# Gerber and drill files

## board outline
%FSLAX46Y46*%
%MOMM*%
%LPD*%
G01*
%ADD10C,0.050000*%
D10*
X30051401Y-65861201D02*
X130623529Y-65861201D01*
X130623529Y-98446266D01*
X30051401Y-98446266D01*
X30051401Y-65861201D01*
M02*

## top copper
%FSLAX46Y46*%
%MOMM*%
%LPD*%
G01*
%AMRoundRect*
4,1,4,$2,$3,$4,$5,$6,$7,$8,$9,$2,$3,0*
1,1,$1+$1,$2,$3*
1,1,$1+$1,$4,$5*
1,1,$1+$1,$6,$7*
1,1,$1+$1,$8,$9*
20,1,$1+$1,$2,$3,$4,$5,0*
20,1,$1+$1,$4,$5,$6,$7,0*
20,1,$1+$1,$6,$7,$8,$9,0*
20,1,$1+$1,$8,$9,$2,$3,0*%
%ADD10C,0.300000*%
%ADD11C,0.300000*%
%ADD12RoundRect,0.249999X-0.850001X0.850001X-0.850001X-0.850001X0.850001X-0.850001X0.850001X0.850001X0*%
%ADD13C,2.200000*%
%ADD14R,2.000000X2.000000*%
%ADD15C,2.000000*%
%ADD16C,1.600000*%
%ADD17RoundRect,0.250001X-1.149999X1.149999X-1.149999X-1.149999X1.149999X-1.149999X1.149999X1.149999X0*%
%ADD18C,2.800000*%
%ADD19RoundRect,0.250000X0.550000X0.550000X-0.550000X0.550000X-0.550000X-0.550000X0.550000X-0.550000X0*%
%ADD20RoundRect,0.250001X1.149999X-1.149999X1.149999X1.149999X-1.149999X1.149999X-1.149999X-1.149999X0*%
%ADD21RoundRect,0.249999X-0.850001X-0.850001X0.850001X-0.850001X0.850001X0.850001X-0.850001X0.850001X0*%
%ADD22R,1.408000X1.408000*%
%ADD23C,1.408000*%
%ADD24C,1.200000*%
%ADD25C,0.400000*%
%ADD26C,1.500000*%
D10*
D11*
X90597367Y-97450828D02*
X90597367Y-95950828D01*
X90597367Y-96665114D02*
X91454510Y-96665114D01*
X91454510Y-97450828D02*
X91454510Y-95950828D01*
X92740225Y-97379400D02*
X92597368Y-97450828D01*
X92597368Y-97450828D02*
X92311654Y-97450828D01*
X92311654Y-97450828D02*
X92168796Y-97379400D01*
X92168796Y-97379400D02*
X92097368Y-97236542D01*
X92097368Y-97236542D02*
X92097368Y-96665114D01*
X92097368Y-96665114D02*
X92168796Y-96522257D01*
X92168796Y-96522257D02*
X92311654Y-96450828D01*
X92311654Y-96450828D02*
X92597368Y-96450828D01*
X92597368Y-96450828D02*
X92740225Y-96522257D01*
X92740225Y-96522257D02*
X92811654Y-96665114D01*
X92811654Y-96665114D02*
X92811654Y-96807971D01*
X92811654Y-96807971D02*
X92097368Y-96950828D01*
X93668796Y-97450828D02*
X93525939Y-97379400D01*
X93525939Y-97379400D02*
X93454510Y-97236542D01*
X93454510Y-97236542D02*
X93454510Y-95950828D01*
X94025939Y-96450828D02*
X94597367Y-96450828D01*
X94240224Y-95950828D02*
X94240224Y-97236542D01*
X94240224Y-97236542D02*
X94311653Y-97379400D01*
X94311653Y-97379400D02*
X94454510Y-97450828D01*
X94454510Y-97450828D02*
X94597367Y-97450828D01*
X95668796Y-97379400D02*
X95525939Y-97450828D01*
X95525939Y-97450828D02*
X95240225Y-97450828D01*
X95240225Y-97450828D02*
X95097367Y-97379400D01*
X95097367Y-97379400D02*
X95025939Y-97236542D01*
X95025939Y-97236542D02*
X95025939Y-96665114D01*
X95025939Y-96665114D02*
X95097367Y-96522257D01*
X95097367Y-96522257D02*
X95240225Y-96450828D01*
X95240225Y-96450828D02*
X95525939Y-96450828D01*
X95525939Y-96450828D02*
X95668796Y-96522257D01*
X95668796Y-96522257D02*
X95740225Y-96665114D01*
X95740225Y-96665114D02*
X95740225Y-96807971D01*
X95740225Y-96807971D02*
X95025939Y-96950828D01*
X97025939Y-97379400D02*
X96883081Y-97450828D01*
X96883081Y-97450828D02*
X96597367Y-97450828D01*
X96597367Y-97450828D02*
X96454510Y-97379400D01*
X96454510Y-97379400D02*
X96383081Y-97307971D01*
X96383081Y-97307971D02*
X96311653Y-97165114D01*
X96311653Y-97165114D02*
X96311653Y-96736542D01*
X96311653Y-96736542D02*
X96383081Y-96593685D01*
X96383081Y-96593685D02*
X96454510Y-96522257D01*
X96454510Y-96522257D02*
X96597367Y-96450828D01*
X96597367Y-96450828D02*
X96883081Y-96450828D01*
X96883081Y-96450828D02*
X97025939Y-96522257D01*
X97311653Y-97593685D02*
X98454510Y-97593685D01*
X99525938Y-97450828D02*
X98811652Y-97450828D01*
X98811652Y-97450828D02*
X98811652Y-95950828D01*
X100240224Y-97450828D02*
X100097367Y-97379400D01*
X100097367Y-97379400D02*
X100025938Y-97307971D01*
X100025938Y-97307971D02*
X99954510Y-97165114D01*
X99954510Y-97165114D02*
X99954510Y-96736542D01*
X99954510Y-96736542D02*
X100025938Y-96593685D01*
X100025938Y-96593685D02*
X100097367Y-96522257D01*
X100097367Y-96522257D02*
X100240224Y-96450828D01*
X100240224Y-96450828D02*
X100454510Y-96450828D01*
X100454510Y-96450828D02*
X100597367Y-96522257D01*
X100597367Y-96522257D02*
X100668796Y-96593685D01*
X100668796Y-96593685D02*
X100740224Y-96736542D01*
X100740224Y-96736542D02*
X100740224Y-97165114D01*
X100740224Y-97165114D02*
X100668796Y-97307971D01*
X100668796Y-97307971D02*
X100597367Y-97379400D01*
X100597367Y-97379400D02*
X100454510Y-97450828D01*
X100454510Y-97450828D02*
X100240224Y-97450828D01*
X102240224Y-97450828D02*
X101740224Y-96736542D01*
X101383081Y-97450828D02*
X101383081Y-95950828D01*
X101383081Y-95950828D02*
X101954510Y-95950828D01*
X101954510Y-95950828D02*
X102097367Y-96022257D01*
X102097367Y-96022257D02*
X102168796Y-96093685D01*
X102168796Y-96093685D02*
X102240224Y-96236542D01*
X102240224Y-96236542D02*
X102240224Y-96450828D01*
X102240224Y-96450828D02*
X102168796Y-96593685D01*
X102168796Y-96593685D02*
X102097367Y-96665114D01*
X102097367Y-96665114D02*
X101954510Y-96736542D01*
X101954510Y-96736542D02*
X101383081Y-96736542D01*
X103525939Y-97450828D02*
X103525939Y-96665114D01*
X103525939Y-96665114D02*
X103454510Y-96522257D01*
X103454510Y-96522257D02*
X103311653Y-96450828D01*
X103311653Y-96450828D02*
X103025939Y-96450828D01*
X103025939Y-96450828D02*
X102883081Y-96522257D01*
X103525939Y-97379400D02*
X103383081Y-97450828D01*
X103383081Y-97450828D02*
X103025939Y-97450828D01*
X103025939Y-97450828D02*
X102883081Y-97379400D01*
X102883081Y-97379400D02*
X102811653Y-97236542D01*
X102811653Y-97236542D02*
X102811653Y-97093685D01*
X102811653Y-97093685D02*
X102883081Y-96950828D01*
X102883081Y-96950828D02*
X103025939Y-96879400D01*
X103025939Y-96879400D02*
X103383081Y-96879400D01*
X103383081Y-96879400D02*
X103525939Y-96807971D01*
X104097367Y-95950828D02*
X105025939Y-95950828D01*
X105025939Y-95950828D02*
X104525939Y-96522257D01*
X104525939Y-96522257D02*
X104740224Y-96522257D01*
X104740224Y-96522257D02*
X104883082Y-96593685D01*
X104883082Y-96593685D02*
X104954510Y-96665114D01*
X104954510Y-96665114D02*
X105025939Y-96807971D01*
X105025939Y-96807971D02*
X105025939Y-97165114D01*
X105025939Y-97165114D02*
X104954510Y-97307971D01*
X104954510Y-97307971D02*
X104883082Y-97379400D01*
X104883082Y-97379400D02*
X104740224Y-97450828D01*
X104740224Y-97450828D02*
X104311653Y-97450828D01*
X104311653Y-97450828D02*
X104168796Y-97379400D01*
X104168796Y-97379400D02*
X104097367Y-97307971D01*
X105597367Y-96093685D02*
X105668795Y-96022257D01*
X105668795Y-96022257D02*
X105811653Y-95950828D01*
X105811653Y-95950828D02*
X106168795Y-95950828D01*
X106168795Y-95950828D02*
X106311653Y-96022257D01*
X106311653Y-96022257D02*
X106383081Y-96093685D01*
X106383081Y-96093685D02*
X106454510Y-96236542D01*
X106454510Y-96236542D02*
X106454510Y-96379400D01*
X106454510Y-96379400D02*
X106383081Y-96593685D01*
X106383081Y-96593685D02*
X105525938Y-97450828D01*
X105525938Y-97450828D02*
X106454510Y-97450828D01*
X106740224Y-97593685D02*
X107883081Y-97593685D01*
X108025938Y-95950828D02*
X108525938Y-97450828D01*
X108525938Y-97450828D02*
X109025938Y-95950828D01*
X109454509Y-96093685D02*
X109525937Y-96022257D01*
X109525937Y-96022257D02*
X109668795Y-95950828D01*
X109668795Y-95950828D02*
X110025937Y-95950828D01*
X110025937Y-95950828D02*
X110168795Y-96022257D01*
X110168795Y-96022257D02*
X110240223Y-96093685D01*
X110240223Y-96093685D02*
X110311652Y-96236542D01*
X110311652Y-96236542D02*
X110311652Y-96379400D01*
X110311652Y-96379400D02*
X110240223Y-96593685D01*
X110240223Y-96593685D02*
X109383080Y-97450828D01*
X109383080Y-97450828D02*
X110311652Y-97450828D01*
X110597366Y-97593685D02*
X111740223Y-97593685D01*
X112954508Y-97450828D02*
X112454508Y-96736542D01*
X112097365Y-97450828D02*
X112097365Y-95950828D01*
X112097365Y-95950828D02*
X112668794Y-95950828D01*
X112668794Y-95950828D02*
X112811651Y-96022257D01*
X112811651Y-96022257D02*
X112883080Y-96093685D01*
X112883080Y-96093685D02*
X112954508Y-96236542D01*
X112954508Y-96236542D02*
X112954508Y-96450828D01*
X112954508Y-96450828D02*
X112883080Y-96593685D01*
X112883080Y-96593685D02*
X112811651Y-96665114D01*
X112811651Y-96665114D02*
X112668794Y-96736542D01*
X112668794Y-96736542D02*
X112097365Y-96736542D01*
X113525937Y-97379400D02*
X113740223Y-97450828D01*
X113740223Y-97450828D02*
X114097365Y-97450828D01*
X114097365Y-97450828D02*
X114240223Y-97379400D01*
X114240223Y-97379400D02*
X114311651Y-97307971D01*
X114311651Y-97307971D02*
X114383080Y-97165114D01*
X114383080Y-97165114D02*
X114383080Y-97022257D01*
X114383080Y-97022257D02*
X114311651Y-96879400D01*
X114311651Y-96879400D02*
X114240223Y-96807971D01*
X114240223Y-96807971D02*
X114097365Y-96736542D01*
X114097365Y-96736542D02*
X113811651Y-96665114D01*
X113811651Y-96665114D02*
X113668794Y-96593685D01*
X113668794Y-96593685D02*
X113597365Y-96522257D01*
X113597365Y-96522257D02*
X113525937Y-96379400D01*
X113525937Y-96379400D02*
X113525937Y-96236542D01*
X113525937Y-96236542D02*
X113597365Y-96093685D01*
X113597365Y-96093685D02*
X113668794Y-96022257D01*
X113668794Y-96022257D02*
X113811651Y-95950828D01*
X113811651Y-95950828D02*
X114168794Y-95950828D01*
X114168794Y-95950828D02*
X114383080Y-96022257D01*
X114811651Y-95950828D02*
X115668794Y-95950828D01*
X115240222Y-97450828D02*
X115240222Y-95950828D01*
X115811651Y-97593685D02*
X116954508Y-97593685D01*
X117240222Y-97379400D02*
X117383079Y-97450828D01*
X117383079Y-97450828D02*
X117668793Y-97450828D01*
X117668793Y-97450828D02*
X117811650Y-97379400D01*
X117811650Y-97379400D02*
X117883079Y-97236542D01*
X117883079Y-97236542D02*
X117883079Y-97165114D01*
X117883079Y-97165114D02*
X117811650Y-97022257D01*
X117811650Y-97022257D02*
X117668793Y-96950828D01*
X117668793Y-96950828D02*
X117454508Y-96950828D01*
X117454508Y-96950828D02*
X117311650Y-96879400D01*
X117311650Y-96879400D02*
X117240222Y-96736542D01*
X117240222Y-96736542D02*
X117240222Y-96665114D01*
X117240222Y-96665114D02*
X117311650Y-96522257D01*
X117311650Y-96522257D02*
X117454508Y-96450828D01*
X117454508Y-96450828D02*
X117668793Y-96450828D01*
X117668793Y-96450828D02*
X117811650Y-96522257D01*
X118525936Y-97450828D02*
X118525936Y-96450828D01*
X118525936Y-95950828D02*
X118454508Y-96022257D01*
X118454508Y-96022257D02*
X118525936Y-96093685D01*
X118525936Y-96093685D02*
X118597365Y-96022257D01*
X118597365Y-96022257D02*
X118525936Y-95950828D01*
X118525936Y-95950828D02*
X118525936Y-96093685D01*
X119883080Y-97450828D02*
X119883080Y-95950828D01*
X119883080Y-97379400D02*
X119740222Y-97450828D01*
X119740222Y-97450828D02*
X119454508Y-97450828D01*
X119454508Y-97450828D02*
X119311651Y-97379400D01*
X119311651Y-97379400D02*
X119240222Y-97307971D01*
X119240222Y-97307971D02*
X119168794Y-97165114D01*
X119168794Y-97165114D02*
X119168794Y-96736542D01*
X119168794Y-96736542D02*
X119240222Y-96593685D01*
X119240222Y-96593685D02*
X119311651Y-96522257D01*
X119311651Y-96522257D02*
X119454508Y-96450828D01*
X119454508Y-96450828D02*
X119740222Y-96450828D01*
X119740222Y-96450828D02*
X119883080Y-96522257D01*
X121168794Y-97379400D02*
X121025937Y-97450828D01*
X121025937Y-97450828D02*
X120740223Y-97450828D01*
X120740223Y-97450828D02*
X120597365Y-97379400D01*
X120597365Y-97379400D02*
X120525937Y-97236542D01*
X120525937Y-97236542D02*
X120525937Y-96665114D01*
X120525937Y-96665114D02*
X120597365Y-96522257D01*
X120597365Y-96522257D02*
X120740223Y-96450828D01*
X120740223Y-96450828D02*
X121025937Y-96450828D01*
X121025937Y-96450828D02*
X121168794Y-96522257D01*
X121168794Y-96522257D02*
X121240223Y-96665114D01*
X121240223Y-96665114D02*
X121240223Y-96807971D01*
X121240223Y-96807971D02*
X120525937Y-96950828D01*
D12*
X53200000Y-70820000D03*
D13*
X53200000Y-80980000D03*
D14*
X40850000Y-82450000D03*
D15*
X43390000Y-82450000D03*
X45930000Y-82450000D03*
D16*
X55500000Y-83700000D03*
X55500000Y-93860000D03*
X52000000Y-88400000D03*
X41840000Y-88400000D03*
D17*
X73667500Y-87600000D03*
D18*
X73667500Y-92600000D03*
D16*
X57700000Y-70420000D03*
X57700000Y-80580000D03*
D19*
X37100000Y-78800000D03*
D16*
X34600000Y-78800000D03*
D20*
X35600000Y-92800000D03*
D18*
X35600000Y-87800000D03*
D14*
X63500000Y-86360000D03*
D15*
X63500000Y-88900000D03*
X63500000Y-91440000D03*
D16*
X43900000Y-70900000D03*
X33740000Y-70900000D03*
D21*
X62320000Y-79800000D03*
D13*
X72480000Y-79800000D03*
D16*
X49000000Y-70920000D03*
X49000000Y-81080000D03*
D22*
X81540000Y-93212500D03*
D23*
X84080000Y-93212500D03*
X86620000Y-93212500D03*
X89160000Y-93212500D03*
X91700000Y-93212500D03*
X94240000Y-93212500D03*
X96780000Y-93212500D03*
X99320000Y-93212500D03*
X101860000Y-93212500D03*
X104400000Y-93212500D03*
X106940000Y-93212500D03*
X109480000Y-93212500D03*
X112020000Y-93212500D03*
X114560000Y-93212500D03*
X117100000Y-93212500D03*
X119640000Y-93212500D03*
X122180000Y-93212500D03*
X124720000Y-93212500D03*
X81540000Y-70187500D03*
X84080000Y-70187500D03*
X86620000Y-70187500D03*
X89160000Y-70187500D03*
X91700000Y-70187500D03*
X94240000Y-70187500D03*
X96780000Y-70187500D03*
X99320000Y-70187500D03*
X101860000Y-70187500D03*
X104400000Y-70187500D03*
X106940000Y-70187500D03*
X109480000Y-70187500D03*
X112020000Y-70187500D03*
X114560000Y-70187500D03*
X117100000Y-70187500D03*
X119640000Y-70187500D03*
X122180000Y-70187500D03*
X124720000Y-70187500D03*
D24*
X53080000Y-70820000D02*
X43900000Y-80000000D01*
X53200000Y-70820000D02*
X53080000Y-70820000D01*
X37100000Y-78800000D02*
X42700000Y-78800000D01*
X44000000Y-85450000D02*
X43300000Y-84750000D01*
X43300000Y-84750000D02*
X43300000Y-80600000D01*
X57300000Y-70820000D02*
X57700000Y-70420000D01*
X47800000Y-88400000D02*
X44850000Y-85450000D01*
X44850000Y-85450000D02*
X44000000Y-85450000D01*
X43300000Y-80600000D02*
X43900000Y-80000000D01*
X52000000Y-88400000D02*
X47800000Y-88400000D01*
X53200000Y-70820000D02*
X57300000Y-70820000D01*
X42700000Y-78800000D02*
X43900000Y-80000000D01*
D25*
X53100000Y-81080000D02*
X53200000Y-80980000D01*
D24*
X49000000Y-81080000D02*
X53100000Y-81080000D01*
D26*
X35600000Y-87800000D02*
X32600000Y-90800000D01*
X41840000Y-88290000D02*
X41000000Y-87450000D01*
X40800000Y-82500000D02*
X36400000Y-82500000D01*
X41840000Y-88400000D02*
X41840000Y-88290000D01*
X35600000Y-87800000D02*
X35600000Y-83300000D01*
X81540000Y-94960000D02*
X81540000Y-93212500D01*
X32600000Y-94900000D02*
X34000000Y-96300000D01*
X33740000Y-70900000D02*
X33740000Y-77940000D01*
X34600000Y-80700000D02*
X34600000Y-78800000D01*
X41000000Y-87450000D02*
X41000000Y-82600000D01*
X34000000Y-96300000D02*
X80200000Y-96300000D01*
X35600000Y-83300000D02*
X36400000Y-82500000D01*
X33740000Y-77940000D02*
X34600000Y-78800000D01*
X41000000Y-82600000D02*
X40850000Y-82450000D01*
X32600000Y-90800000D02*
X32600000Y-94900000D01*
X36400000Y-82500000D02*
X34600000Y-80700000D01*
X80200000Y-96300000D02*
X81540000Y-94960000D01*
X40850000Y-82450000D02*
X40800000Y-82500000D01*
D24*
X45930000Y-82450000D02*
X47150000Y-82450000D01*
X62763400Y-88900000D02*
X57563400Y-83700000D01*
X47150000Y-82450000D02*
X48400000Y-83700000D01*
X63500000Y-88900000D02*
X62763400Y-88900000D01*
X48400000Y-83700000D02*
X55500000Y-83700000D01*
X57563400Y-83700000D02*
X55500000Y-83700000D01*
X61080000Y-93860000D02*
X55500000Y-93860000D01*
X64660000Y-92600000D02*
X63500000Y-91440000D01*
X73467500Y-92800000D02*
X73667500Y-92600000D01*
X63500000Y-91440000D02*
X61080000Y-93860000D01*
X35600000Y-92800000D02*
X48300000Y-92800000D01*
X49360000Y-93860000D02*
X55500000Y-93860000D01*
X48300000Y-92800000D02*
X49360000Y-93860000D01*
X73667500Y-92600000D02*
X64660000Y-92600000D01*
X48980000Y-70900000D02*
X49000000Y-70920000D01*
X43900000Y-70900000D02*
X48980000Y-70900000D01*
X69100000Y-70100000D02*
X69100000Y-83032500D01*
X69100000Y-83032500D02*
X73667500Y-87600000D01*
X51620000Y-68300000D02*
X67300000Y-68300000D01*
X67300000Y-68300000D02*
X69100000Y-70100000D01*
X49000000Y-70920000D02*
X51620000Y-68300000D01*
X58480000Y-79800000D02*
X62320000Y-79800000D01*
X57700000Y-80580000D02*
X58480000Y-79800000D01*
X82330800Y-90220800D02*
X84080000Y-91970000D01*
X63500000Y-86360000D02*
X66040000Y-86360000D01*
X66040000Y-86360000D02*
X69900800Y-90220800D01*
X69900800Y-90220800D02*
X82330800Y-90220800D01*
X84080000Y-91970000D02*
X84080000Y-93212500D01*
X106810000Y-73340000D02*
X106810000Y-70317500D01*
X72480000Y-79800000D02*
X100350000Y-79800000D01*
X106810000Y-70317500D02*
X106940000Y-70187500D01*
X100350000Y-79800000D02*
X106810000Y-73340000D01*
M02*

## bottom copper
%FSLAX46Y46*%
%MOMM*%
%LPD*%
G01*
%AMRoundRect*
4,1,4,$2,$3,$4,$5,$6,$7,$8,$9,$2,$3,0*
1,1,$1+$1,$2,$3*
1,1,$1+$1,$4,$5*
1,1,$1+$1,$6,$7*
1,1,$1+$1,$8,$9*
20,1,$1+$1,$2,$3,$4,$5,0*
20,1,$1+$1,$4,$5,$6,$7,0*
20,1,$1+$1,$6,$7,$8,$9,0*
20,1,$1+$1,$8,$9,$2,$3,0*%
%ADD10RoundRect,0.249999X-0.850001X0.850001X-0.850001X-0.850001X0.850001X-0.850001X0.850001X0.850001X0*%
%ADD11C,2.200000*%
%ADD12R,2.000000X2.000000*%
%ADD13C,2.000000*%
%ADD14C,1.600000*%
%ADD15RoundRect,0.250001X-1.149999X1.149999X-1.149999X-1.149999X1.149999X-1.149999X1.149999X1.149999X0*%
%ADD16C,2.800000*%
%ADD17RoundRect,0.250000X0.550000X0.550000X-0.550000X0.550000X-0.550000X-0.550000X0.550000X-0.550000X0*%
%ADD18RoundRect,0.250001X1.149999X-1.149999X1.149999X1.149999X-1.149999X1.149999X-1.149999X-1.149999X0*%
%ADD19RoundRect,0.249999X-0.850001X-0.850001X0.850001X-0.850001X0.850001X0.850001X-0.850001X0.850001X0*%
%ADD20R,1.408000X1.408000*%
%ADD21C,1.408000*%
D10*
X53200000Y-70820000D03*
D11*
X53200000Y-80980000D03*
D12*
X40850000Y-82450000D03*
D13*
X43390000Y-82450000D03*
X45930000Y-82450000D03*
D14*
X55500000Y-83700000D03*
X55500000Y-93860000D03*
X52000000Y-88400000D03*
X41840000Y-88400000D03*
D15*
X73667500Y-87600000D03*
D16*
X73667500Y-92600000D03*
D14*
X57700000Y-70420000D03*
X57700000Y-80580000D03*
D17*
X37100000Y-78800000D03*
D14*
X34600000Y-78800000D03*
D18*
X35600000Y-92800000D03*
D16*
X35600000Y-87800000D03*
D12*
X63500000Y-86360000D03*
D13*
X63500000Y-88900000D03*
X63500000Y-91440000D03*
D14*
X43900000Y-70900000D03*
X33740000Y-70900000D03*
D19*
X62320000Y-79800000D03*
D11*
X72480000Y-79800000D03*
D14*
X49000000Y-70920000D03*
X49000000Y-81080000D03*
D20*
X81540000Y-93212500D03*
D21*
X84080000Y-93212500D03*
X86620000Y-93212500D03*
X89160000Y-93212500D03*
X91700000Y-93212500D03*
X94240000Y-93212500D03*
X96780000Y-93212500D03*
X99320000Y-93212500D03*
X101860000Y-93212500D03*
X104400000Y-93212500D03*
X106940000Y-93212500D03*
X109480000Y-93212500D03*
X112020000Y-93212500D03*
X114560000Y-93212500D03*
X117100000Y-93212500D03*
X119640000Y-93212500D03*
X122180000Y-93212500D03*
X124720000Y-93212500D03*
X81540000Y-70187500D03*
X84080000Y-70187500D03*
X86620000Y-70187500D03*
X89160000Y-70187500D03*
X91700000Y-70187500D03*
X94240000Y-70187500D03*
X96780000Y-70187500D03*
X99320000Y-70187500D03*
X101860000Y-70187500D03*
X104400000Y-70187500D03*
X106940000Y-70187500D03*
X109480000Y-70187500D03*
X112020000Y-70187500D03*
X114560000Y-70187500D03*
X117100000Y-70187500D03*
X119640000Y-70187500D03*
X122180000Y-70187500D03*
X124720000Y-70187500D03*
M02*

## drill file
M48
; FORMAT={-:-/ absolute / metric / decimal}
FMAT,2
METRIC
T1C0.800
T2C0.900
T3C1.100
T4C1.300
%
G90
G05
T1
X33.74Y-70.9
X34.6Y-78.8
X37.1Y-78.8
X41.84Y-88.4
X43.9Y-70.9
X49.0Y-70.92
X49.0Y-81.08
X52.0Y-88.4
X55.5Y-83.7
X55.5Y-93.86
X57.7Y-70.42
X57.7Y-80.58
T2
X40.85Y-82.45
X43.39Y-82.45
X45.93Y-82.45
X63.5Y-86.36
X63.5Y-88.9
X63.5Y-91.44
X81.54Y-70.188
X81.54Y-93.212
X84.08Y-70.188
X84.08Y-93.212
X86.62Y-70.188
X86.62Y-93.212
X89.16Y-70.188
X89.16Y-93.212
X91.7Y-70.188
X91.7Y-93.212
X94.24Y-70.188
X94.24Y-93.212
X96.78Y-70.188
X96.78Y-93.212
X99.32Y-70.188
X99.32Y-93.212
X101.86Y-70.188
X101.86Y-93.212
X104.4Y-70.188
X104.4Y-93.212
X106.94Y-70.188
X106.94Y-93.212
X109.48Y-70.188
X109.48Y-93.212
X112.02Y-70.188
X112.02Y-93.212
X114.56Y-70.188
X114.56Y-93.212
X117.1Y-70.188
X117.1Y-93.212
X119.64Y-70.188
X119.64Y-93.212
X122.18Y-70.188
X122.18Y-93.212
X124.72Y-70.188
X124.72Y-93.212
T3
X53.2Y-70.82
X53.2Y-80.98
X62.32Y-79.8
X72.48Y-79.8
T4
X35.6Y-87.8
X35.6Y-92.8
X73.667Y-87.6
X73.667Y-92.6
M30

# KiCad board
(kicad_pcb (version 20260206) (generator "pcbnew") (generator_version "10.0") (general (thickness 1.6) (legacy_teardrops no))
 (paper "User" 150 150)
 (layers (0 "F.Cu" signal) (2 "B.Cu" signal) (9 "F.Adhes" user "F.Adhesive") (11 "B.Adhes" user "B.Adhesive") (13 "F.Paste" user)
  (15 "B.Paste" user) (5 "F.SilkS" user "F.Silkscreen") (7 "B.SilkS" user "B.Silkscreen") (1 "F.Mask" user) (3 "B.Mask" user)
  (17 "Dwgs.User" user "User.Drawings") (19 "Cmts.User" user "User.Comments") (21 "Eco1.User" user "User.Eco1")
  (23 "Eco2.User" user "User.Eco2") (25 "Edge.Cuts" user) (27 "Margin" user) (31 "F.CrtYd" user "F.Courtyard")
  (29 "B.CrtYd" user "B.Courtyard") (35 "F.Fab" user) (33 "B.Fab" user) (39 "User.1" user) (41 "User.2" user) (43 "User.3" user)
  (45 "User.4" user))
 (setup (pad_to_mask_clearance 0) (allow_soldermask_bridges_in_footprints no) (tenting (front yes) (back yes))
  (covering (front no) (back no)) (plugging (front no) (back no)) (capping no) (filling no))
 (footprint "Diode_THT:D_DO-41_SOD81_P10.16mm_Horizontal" (layer "F.Cu") (at 53.2 70.82 -90)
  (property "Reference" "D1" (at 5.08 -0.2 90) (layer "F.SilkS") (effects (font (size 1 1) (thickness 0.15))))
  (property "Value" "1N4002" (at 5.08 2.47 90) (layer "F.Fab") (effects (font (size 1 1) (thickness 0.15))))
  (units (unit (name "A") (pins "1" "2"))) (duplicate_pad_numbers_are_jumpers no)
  (pad "1" thru_hole roundrect (at 0 0 270) (size 2.2 2.2) (drill 1.1) (layers "*.Cu" "*.Mask") (remove_unused_layers no)
   (roundrect_rratio 0.113636) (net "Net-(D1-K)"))
  (pad "2" thru_hole circle (at 10.16 0 270) (size 2.2 2.2) (drill 1.1) (layers "*.Cu" "*.Mask") (remove_unused_layers no)
   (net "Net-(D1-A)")))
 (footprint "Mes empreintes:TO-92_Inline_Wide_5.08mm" (layer "F.Cu") (at 40.85 82.45)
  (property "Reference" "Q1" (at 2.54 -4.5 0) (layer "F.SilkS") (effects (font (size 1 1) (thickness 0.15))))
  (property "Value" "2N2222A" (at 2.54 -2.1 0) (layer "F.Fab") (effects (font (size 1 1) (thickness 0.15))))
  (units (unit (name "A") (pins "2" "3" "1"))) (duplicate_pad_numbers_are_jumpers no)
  (pad "1" thru_hole rect (at 0 0) (size 2 2) (drill 0.9) (layers "*.Cu" "*.Mask") (remove_unused_layers no) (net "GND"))
  (pad "2" thru_hole circle (at 2.54 0) (size 2 2) (drill 0.9) (layers "*.Cu" "*.Mask") (remove_unused_layers no) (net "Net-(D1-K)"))
  (pad "3" thru_hole circle (at 5.08 0) (size 2 2) (drill 0.9) (layers "*.Cu" "*.Mask") (remove_unused_layers no) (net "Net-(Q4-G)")))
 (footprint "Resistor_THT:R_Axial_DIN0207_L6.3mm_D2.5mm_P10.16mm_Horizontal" (layer "F.Cu") (at 55.5 83.7 -90)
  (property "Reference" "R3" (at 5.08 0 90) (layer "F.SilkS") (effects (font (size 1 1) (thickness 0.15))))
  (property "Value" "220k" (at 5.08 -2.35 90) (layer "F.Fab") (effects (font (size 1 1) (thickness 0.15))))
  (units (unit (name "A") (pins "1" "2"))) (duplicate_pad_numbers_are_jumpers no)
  (pad "1" thru_hole circle (at 0 0 270) (size 1.6 1.6) (drill 0.8) (layers "*.Cu" "*.Mask") (remove_unused_layers no) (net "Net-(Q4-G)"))
  (pad "2" thru_hole circle (at 10.16 0 270) (size 1.6 1.6) (drill 0.8) (layers "*.Cu" "*.Mask") (remove_unused_layers no) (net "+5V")))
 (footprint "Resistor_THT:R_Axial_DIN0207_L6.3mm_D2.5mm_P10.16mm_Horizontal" (layer "F.Cu") (at 52 88.4 180)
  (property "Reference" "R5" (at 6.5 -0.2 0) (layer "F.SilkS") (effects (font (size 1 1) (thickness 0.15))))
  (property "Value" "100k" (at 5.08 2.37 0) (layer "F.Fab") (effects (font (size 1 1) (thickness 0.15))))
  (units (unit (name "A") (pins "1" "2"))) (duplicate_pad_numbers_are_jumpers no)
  (pad "1" thru_hole circle (at 0 0 180) (size 1.6 1.6) (drill 0.8) (layers "*.Cu" "*.Mask") (remove_unused_layers no) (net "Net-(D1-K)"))
  (pad "2" thru_hole circle (at 10.16 0 180) (size 1.6 1.6) (drill 0.8) (layers "*.Cu" "*.Mask") (remove_unused_layers no) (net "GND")))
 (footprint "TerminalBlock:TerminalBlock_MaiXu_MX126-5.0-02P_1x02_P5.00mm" (layer "F.Cu") (at 73.6675 87.6 -90)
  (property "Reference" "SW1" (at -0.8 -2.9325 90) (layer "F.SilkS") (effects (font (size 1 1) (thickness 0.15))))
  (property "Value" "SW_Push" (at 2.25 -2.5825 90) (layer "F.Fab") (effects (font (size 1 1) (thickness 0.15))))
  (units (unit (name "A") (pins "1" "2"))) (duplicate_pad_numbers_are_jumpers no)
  (pad "1" thru_hole roundrect (at 0 0 270) (size 2.8 2.8) (drill 1.3) (layers "*.Cu" "*.Mask") (remove_unused_layers no)
   (roundrect_rratio 0.089286) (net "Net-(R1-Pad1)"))
  (pad "2" thru_hole circle (at 5 0 270) (size 2.8 2.8) (drill 1.3) (layers "*.Cu" "*.Mask") (remove_unused_layers no) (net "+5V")))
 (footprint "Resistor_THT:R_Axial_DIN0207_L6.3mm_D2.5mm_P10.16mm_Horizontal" (layer "F.Cu") (at 57.7 70.42 -90)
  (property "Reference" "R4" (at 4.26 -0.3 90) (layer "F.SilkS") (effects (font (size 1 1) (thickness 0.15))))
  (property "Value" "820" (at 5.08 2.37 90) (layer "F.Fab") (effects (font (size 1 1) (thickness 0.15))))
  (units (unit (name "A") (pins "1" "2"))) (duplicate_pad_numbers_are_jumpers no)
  (pad "1" thru_hole circle (at 0 0 270) (size 1.6 1.6) (drill 0.8) (layers "*.Cu" "*.Mask") (remove_unused_layers no) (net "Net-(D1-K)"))
  (pad "2" thru_hole circle (at 10.16 0 270) (size 1.6 1.6) (drill 0.8) (layers "*.Cu" "*.Mask") (remove_unused_layers no)
   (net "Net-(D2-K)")))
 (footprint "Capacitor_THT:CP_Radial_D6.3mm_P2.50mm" (layer "F.Cu") (at 37.1 78.8 180)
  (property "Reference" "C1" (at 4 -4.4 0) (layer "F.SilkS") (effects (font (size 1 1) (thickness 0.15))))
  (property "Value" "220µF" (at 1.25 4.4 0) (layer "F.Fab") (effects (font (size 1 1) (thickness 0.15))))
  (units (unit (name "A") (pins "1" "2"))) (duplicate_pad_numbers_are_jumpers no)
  (pad "1" thru_hole roundrect (at 0 0 180) (size 1.6 1.6) (drill 0.8) (layers "*.Cu" "*.Mask") (remove_unused_layers no)
   (roundrect_rratio 0.15625) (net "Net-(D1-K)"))
  (pad "2" thru_hole circle (at 2.5 0 180) (size 1.6 1.6) (drill 0.8) (layers "*.Cu" "*.Mask") (remove_unused_layers no) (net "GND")))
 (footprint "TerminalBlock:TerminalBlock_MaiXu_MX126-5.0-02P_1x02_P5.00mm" (layer "F.Cu") (at 35.6 92.8 90)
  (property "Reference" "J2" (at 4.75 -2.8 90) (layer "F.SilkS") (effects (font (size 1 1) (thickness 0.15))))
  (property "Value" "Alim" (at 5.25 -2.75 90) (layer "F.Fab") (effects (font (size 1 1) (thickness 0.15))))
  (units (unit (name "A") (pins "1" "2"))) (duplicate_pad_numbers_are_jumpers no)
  (pad "1" thru_hole roundrect (at 0 0 90) (size 2.8 2.8) (drill 1.3) (layers "*.Cu" "*.Mask") (remove_unused_layers no)
   (roundrect_rratio 0.089286) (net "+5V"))
  (pad "2" thru_hole circle (at 5 0 90) (size 2.8 2.8) (drill 1.3) (layers "*.Cu" "*.Mask") (remove_unused_layers no) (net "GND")))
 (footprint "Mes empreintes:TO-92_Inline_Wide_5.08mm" (layer "F.Cu") (at 63.5 86.36 -90)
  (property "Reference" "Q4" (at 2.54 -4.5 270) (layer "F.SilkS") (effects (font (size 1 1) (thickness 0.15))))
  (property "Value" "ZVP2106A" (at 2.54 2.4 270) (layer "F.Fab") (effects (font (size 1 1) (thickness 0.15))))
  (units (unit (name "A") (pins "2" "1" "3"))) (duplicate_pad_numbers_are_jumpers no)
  (pad "1" thru_hole rect (at 0 0 270) (size 2 2) (drill 0.9) (layers "*.Cu" "*.Mask") (remove_unused_layers no) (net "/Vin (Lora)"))
  (pad "2" thru_hole circle (at 2.54 0 270) (size 2 2) (drill 0.9) (layers "*.Cu" "*.Mask") (remove_unused_layers no) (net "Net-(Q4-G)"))
  (pad "3" thru_hole circle (at 5.08 0 270) (size 2 2) (drill 0.9) (layers "*.Cu" "*.Mask") (remove_unused_layers no) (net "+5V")))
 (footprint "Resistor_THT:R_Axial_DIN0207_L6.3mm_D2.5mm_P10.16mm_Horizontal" (layer "F.Cu") (at 43.9 70.9 180)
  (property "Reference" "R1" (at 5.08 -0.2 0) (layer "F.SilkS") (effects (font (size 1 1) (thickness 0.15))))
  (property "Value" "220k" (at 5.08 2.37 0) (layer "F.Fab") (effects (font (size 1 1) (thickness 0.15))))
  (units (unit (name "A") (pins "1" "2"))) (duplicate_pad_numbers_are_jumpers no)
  (pad "1" thru_hole circle (at 0 0 180) (size 1.6 1.6) (drill 0.8) (layers "*.Cu" "*.Mask") (remove_unused_layers no) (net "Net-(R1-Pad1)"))
  (pad "2" thru_hole circle (at 10.16 0 180) (size 1.6 1.6) (drill 0.8) (layers "*.Cu" "*.Mask") (remove_unused_layers no) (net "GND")))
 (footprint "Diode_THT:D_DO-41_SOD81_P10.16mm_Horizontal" (layer "F.Cu") (at 62.32 79.8)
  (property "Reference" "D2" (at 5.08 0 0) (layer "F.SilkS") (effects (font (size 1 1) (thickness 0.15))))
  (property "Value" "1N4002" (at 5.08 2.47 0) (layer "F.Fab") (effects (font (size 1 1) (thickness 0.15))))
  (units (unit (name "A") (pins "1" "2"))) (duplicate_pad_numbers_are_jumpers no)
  (pad "1" thru_hole roundrect (at 0 0) (size 2.2 2.2) (drill 1.1) (layers "*.Cu" "*.Mask") (remove_unused_layers no)
   (roundrect_rratio 0.113636) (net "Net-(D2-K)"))
  (pad "2" thru_hole circle (at 10.16 0) (size 2.2 2.2) (drill 1.1) (layers "*.Cu" "*.Mask") (remove_unused_layers no)
   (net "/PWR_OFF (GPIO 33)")))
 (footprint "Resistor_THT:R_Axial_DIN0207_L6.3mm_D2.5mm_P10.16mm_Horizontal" (layer "F.Cu") (at 49 70.92 -90)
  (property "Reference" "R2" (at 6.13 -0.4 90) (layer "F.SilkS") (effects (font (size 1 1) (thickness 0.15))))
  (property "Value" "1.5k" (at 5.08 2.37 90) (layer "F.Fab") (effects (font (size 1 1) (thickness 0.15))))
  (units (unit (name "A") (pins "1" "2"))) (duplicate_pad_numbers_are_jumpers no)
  (pad "1" thru_hole circle (at 0 0 270) (size 1.6 1.6) (drill 0.8) (layers "*.Cu" "*.Mask") (remove_unused_layers no) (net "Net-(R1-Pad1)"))
  (pad "2" thru_hole circle (at 10.16 0 270) (size 1.6 1.6) (drill 0.8) (layers "*.Cu" "*.Mask") (remove_unused_layers no)
   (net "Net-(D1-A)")))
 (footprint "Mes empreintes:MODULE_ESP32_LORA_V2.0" (layer "F.Cu") (at 103.92 81.7)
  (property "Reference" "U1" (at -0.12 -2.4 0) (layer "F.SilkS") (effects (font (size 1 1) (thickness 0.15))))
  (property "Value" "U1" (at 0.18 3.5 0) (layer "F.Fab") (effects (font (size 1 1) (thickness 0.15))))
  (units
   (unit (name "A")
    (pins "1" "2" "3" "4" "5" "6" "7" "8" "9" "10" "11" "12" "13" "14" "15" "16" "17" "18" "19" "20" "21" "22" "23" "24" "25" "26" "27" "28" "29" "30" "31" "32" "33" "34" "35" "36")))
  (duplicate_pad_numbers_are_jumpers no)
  (pad "1" thru_hole rect (at -22.38 11.5125) (size 1.408 1.408) (drill 0.9) (layers "*.Cu" "*.Mask") (remove_unused_layers no) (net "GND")
   (solder_mask_margin 0.102))
  (pad "2" thru_hole circle (at -19.84 11.5125) (size 1.408 1.408) (drill 0.9) (layers "*.Cu" "*.Mask") (remove_unused_layers no)
   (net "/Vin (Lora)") (solder_mask_margin 0.102))
  (pad "3" thru_hole circle (at -17.3 11.5125) (size 1.408 1.408) (drill 0.9) (layers "*.Cu" "*.Mask") (remove_unused_layers no)
   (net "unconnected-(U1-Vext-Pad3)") (solder_mask_margin 0.102))
  (pad "4" thru_hole circle (at -14.76 11.5125) (size 1.408 1.408) (drill 0.9) (layers "*.Cu" "*.Mask") (remove_unused_layers no)
   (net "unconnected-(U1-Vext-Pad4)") (solder_mask_margin 0.102))
  (pad "5" thru_hole circle (at -12.22 11.5125) (size 1.408 1.408) (drill 0.9) (layers "*.Cu" "*.Mask") (remove_unused_layers no)
   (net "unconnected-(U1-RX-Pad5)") (solder_mask_margin 0.102))
  (pad "6" thru_hole circle (at -9.68 11.5125) (size 1.408 1.408) (drill 0.9) (layers "*.Cu" "*.Mask") (remove_unused_layers no)
   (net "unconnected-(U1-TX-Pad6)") (solder_mask_margin 0.102))
  (pad "7" thru_hole circle (at -7.14 11.5125) (size 1.408 1.408) (drill 0.9) (layers "*.Cu" "*.Mask") (remove_unused_layers no)
   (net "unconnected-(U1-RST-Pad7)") (solder_mask_margin 0.102))
  (pad "8" thru_hole circle (at -4.6 11.5125) (size 1.408 1.408) (drill 0.9) (layers "*.Cu" "*.Mask") (remove_unused_layers no)
   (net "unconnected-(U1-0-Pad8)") (solder_mask_margin 0.102))
  (pad "9" thru_hole circle (at -2.06 11.5125) (size 1.408 1.408) (drill 0.9) (layers "*.Cu" "*.Mask") (remove_unused_layers no)
   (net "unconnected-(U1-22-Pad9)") (solder_mask_margin 0.102))
  (pad "10" thru_hole circle (at 0.48 11.5125) (size 1.408 1.408) (drill 0.9) (layers "*.Cu" "*.Mask") (remove_unused_layers no)
   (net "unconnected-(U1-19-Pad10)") (solder_mask_margin 0.102))
  (pad "11" thru_hole circle (at 3.02 11.5125) (size 1.408 1.408) (drill 0.9) (layers "*.Cu" "*.Mask") (remove_unused_layers no)
   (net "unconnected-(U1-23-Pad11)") (solder_mask_margin 0.102))
  (pad "12" thru_hole circle (at 5.56 11.5125) (size 1.408 1.408) (drill 0.9) (layers "*.Cu" "*.Mask") (remove_unused_layers no)
   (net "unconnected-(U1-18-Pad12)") (solder_mask_margin 0.102))
  (pad "13" thru_hole circle (at 8.1 11.5125) (size 1.408 1.408) (drill 0.9) (layers "*.Cu" "*.Mask") (remove_unused_layers no)
   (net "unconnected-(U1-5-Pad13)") (solder_mask_margin 0.102))
  (pad "14" thru_hole circle (at 10.64 11.5125) (size 1.408 1.408) (drill 0.9) (layers "*.Cu" "*.Mask") (remove_unused_layers no)
   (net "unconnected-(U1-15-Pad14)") (solder_mask_margin 0.102))
  (pad "15" thru_hole circle (at 13.18 11.5125) (size 1.408 1.408) (drill 0.9) (layers "*.Cu" "*.Mask") (remove_unused_layers no)
   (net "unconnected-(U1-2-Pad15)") (solder_mask_margin 0.102))
  (pad "16" thru_hole circle (at 15.72 11.5125) (size 1.408 1.408) (drill 0.9) (layers "*.Cu" "*.Mask") (remove_unused_layers no)
   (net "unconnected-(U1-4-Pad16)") (solder_mask_margin 0.102))
  (pad "17" thru_hole circle (at 18.26 11.5125) (size 1.408 1.408) (drill 0.9) (layers "*.Cu" "*.Mask") (remove_unused_layers no)
   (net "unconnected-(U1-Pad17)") (solder_mask_margin 0.102))
  (pad "18" thru_hole circle (at 20.8 11.5125) (size 1.408 1.408) (drill 0.9) (layers "*.Cu" "*.Mask") (remove_unused_layers no)
   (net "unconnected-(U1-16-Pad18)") (solder_mask_margin 0.102))
  (pad "19" thru_hole circle (at -22.38 -11.5125) (size 1.408 1.408) (drill 0.9) (layers "*.Cu" "*.Mask") (remove_unused_layers no)
   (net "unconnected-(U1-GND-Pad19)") (solder_mask_margin 0.102))
  (pad "20" thru_hole circle (at -19.84 -11.5125) (size 1.408 1.408) (drill 0.9) (layers "*.Cu" "*.Mask") (remove_unused_layers no)
   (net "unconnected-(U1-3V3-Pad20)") (solder_mask_margin 0.102))
  (pad "21" thru_hole circle (at -17.3 -11.5125) (size 1.408 1.408) (drill 0.9) (layers "*.Cu" "*.Mask") (remove_unused_layers no)
   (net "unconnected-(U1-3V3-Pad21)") (solder_mask_margin 0.102))
  (pad "22" thru_hole circle (at -14.76 -11.5125) (size 1.408 1.408) (drill 0.9) (layers "*.Cu" "*.Mask") (remove_unused_layers no)
   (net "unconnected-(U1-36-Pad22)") (solder_mask_margin 0.102))
  (pad "23" thru_hole circle (at -12.22 -11.5125) (size 1.408 1.408) (drill 0.9) (layers "*.Cu" "*.Mask") (remove_unused_layers no)
   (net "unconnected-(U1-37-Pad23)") (solder_mask_margin 0.102))
  (pad "24" thru_hole circle (at -9.68 -11.5125) (size 1.408 1.408) (drill 0.9) (layers "*.Cu" "*.Mask") (remove_unused_layers no)
   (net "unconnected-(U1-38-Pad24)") (solder_mask_margin 0.102))
  (pad "25" thru_hole circle (at -7.14 -11.5125) (size 1.408 1.408) (drill 0.9) (layers "*.Cu" "*.Mask") (remove_unused_layers no)
   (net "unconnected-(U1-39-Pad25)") (solder_mask_margin 0.102))
  (pad "26" thru_hole circle (at -4.6 -11.5125) (size 1.408 1.408) (drill 0.9) (layers "*.Cu" "*.Mask") (remove_unused_layers no)
   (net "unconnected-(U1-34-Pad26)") (solder_mask_margin 0.102))
  (pad "27" thru_hole circle (at -2.06 -11.5125) (size 1.408 1.408) (drill 0.9) (layers "*.Cu" "*.Mask") (remove_unused_layers no)
   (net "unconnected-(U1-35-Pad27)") (solder_mask_margin 0.102))
  (pad "28" thru_hole circle (at 0.48 -11.5125) (size 1.408 1.408) (drill 0.9) (layers "*.Cu" "*.Mask") (remove_unused_layers no)
   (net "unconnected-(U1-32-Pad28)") (solder_mask_margin 0.102))
  (pad "29" thru_hole circle (at 3.02 -11.5125) (size 1.408 1.408) (drill 0.9) (layers "*.Cu" "*.Mask") (remove_unused_layers no)
   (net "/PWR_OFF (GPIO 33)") (solder_mask_margin 0.102))
  (pad "30" thru_hole circle (at 5.56 -11.5125) (size 1.408 1.408) (drill 0.9) (layers "*.Cu" "*.Mask") (remove_unused_layers no)
   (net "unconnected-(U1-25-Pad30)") (solder_mask_margin 0.102))
  (pad "31" thru_hole circle (at 8.1 -11.5125) (size 1.408 1.408) (drill 0.9) (layers "*.Cu" "*.Mask") (remove_unused_layers no)
   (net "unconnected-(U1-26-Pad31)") (solder_mask_margin 0.102))
  (pad "32" thru_hole circle (at 10.64 -11.5125) (size 1.408 1.408) (drill 0.9) (layers "*.Cu" "*.Mask") (remove_unused_layers no)
   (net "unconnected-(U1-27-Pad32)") (solder_mask_margin 0.102))
  (pad "33" thru_hole circle (at 13.18 -11.5125) (size 1.408 1.408) (drill 0.9) (layers "*.Cu" "*.Mask") (remove_unused_layers no)
   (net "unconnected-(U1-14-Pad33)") (solder_mask_margin 0.102))
  (pad "34" thru_hole circle (at 15.72 -11.5125) (size 1.408 1.408) (drill 0.9) (layers "*.Cu" "*.Mask") (remove_unused_layers no)
   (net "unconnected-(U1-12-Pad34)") (solder_mask_margin 0.102))
  (pad "35" thru_hole circle (at 18.26 -11.5125) (size 1.408 1.408) (drill 0.9) (layers "*.Cu" "*.Mask") (remove_unused_layers no)
   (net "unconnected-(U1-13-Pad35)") (solder_mask_margin 0.102))
  (pad "36" thru_hole circle (at 20.8 -11.5125) (size 1.408 1.408) (drill 0.9) (layers "*.Cu" "*.Mask") (remove_unused_layers no)
   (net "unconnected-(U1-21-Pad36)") (solder_mask_margin 0.102)))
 (gr_rect (start 30.051401 65.861201) (end 130.623529 98.446266) (stroke (width 0.05) (type default)) (fill no) (layer "Edge.Cuts"))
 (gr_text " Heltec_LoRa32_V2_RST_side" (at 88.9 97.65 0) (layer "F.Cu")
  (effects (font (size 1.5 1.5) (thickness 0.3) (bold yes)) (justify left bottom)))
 (segment (start 53.08 70.82) (end 43.9 80) (width 1.2) (layer "F.Cu") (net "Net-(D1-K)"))
 (segment (start 53.2 70.82) (end 53.08 70.82) (width 1.2) (layer "F.Cu") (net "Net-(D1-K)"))
 (segment (start 37.1 78.8) (end 42.7 78.8) (width 1.2) (layer "F.Cu") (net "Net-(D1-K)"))
 (segment (start 44 85.45) (end 43.3 84.75) (width 1.2) (layer "F.Cu") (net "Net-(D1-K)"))
 (segment (start 43.3 84.75) (end 43.3 80.6) (width 1.2) (layer "F.Cu") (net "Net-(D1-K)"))
 (segment (start 57.3 70.82) (end 57.7 70.42) (width 1.2) (layer "F.Cu") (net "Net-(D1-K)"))
 (segment (start 47.8 88.4) (end 44.85 85.45) (width 1.2) (layer "F.Cu") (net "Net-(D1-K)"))
 (segment (start 44.85 85.45) (end 44 85.45) (width 1.2) (layer "F.Cu") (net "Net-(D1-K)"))
 (segment (start 43.3 80.6) (end 43.9 80) (width 1.2) (layer "F.Cu") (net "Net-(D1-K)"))
 (segment (start 52 88.4) (end 47.8 88.4) (width 1.2) (layer "F.Cu") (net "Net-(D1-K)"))
 (segment (start 53.2 70.82) (end 57.3 70.82) (width 1.2) (layer "F.Cu") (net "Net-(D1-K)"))
 (segment (start 42.7 78.8) (end 43.9 80) (width 1.2) (layer "F.Cu") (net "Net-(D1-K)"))
 (segment (start 53.1 81.08) (end 53.2 80.98) (width 0.4) (layer "F.Cu") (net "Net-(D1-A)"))
 (segment (start 49 81.08) (end 53.1 81.08) (width 1.2) (layer "F.Cu") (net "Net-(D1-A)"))
 (segment (start 35.6 87.8) (end 32.6 90.8) (width 1.5) (layer "F.Cu") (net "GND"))
 (segment (start 41.84 88.29) (end 41 87.45) (width 1.5) (layer "F.Cu") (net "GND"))
 (segment (start 40.8 82.5) (end 36.4 82.5) (width 1.5) (layer "F.Cu") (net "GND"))
 (segment (start 41.84 88.4) (end 41.84 88.29) (width 1.5) (layer "F.Cu") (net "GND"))
 (segment (start 35.6 87.8) (end 35.6 83.3) (width 1.5) (layer "F.Cu") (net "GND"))
 (segment (start 81.54 94.96) (end 81.54 93.2125) (width 1.5) (layer "F.Cu") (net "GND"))
 (segment (start 32.6 94.9) (end 34 96.3) (width 1.5) (layer "F.Cu") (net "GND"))
 (segment (start 33.74 70.9) (end 33.74 77.94) (width 1.5) (layer "F.Cu") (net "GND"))
 (segment (start 34.6 80.7) (end 34.6 78.8) (width 1.5) (layer "F.Cu") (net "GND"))
 (segment (start 41 87.45) (end 41 82.6) (width 1.5) (layer "F.Cu") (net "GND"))
 (segment (start 34 96.3) (end 80.2 96.3) (width 1.5) (layer "F.Cu") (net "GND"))
 (segment (start 35.6 83.3) (end 36.4 82.5) (width 1.5) (layer "F.Cu") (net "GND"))
 (segment (start 33.74 77.94) (end 34.6 78.8) (width 1.5) (layer "F.Cu") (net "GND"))
 (segment (start 41 82.6) (end 40.85 82.45) (width 1.5) (layer "F.Cu") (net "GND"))
 (segment (start 32.6 90.8) (end 32.6 94.9) (width 1.5) (layer "F.Cu") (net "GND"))
 (segment (start 36.4 82.5) (end 34.6 80.7) (width 1.5) (layer "F.Cu") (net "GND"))
 (segment (start 80.2 96.3) (end 81.54 94.96) (width 1.5) (layer "F.Cu") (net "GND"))
 (segment (start 40.85 82.45) (end 40.8 82.5) (width 1.5) (layer "F.Cu") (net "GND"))
 (segment (start 45.93 82.45) (end 47.15 82.45) (width 1.2) (layer "F.Cu") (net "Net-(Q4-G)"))
 (segment (start 62.7634 88.9) (end 57.5634 83.7) (width 1.2) (layer "F.Cu") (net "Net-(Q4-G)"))
 (segment (start 47.15 82.45) (end 48.4 83.7) (width 1.2) (layer "F.Cu") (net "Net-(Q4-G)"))
 (segment (start 63.5 88.9) (end 62.7634 88.9) (width 1.2) (layer "F.Cu") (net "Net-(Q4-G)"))
 (segment (start 48.4 83.7) (end 55.5 83.7) (width 1.2) (layer "F.Cu") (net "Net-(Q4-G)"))
 (segment (start 57.5634 83.7) (end 55.5 83.7) (width 1.2) (layer "F.Cu") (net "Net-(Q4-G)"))
 (segment (start 61.08 93.86) (end 55.5 93.86) (width 1.2) (layer "F.Cu") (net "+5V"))
 (segment (start 64.66 92.6) (end 63.5 91.44) (width 1.2) (layer "F.Cu") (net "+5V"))
 (segment (start 73.4675 92.8) (end 73.6675 92.6) (width 1.2) (layer "F.Cu") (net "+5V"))
 (segment (start 63.5 91.44) (end 61.08 93.86) (width 1.2) (layer "F.Cu") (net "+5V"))
 (segment (start 35.6 92.8) (end 48.3 92.8) (width 1.2) (layer "F.Cu") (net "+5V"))
 (segment (start 49.36 93.86) (end 55.5 93.86) (width 1.2) (layer "F.Cu") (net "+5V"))
 (segment (start 48.3 92.8) (end 49.36 93.86) (width 1.2) (layer "F.Cu") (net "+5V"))
 (segment (start 73.6675 92.6) (end 64.66 92.6) (width 1.2) (layer "F.Cu") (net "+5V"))
 (segment (start 48.98 70.9) (end 49 70.92) (width 1.2) (layer "F.Cu") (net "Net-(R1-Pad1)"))
 (segment (start 43.9 70.9) (end 48.98 70.9) (width 1.2) (layer "F.Cu") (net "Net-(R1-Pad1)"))
 (segment (start 69.1 70.1) (end 69.1 83.0325) (width 1.2) (layer "F.Cu") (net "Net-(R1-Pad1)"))
 (segment (start 69.1 83.0325) (end 73.6675 87.6) (width 1.2) (layer "F.Cu") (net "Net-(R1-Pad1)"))
 (segment (start 51.62 68.3) (end 67.3 68.3) (width 1.2) (layer "F.Cu") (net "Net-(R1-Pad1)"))
 (segment (start 67.3 68.3) (end 69.1 70.1) (width 1.2) (layer "F.Cu") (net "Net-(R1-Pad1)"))
 (segment (start 49 70.92) (end 51.62 68.3) (width 1.2) (layer "F.Cu") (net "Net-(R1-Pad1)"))
 (segment (start 58.48 79.8) (end 62.32 79.8) (width 1.2) (layer "F.Cu") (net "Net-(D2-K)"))
 (segment (start 57.7 80.58) (end 58.48 79.8) (width 1.2) (layer "F.Cu") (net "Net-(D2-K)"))
 (segment (start 82.3308 90.2208) (end 84.08 91.97) (width 1.2) (layer "F.Cu") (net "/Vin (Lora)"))
 (segment (start 63.5 86.36) (end 66.04 86.36) (width 1.2) (layer "F.Cu") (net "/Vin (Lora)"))
 (segment (start 66.04 86.36) (end 69.9008 90.2208) (width 1.2) (layer "F.Cu") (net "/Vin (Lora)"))
 (segment (start 69.9008 90.2208) (end 82.3308 90.2208) (width 1.2) (layer "F.Cu") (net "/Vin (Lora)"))
 (segment (start 84.08 91.97) (end 84.08 93.2125) (width 1.2) (layer "F.Cu") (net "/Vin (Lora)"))
 (segment (start 106.81 73.34) (end 106.81 70.3175) (width 1.2) (layer "F.Cu") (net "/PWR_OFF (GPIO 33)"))
 (segment (start 72.48 79.8) (end 100.35 79.8) (width 1.2) (layer "F.Cu") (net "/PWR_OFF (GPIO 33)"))
 (segment (start 106.81 70.3175) (end 106.94 70.1875) (width 1.2) (layer "F.Cu") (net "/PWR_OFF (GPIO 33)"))
 (segment (start 100.35 79.8) (end 106.81 73.34) (width 1.2) (layer "F.Cu") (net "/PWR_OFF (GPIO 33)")))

